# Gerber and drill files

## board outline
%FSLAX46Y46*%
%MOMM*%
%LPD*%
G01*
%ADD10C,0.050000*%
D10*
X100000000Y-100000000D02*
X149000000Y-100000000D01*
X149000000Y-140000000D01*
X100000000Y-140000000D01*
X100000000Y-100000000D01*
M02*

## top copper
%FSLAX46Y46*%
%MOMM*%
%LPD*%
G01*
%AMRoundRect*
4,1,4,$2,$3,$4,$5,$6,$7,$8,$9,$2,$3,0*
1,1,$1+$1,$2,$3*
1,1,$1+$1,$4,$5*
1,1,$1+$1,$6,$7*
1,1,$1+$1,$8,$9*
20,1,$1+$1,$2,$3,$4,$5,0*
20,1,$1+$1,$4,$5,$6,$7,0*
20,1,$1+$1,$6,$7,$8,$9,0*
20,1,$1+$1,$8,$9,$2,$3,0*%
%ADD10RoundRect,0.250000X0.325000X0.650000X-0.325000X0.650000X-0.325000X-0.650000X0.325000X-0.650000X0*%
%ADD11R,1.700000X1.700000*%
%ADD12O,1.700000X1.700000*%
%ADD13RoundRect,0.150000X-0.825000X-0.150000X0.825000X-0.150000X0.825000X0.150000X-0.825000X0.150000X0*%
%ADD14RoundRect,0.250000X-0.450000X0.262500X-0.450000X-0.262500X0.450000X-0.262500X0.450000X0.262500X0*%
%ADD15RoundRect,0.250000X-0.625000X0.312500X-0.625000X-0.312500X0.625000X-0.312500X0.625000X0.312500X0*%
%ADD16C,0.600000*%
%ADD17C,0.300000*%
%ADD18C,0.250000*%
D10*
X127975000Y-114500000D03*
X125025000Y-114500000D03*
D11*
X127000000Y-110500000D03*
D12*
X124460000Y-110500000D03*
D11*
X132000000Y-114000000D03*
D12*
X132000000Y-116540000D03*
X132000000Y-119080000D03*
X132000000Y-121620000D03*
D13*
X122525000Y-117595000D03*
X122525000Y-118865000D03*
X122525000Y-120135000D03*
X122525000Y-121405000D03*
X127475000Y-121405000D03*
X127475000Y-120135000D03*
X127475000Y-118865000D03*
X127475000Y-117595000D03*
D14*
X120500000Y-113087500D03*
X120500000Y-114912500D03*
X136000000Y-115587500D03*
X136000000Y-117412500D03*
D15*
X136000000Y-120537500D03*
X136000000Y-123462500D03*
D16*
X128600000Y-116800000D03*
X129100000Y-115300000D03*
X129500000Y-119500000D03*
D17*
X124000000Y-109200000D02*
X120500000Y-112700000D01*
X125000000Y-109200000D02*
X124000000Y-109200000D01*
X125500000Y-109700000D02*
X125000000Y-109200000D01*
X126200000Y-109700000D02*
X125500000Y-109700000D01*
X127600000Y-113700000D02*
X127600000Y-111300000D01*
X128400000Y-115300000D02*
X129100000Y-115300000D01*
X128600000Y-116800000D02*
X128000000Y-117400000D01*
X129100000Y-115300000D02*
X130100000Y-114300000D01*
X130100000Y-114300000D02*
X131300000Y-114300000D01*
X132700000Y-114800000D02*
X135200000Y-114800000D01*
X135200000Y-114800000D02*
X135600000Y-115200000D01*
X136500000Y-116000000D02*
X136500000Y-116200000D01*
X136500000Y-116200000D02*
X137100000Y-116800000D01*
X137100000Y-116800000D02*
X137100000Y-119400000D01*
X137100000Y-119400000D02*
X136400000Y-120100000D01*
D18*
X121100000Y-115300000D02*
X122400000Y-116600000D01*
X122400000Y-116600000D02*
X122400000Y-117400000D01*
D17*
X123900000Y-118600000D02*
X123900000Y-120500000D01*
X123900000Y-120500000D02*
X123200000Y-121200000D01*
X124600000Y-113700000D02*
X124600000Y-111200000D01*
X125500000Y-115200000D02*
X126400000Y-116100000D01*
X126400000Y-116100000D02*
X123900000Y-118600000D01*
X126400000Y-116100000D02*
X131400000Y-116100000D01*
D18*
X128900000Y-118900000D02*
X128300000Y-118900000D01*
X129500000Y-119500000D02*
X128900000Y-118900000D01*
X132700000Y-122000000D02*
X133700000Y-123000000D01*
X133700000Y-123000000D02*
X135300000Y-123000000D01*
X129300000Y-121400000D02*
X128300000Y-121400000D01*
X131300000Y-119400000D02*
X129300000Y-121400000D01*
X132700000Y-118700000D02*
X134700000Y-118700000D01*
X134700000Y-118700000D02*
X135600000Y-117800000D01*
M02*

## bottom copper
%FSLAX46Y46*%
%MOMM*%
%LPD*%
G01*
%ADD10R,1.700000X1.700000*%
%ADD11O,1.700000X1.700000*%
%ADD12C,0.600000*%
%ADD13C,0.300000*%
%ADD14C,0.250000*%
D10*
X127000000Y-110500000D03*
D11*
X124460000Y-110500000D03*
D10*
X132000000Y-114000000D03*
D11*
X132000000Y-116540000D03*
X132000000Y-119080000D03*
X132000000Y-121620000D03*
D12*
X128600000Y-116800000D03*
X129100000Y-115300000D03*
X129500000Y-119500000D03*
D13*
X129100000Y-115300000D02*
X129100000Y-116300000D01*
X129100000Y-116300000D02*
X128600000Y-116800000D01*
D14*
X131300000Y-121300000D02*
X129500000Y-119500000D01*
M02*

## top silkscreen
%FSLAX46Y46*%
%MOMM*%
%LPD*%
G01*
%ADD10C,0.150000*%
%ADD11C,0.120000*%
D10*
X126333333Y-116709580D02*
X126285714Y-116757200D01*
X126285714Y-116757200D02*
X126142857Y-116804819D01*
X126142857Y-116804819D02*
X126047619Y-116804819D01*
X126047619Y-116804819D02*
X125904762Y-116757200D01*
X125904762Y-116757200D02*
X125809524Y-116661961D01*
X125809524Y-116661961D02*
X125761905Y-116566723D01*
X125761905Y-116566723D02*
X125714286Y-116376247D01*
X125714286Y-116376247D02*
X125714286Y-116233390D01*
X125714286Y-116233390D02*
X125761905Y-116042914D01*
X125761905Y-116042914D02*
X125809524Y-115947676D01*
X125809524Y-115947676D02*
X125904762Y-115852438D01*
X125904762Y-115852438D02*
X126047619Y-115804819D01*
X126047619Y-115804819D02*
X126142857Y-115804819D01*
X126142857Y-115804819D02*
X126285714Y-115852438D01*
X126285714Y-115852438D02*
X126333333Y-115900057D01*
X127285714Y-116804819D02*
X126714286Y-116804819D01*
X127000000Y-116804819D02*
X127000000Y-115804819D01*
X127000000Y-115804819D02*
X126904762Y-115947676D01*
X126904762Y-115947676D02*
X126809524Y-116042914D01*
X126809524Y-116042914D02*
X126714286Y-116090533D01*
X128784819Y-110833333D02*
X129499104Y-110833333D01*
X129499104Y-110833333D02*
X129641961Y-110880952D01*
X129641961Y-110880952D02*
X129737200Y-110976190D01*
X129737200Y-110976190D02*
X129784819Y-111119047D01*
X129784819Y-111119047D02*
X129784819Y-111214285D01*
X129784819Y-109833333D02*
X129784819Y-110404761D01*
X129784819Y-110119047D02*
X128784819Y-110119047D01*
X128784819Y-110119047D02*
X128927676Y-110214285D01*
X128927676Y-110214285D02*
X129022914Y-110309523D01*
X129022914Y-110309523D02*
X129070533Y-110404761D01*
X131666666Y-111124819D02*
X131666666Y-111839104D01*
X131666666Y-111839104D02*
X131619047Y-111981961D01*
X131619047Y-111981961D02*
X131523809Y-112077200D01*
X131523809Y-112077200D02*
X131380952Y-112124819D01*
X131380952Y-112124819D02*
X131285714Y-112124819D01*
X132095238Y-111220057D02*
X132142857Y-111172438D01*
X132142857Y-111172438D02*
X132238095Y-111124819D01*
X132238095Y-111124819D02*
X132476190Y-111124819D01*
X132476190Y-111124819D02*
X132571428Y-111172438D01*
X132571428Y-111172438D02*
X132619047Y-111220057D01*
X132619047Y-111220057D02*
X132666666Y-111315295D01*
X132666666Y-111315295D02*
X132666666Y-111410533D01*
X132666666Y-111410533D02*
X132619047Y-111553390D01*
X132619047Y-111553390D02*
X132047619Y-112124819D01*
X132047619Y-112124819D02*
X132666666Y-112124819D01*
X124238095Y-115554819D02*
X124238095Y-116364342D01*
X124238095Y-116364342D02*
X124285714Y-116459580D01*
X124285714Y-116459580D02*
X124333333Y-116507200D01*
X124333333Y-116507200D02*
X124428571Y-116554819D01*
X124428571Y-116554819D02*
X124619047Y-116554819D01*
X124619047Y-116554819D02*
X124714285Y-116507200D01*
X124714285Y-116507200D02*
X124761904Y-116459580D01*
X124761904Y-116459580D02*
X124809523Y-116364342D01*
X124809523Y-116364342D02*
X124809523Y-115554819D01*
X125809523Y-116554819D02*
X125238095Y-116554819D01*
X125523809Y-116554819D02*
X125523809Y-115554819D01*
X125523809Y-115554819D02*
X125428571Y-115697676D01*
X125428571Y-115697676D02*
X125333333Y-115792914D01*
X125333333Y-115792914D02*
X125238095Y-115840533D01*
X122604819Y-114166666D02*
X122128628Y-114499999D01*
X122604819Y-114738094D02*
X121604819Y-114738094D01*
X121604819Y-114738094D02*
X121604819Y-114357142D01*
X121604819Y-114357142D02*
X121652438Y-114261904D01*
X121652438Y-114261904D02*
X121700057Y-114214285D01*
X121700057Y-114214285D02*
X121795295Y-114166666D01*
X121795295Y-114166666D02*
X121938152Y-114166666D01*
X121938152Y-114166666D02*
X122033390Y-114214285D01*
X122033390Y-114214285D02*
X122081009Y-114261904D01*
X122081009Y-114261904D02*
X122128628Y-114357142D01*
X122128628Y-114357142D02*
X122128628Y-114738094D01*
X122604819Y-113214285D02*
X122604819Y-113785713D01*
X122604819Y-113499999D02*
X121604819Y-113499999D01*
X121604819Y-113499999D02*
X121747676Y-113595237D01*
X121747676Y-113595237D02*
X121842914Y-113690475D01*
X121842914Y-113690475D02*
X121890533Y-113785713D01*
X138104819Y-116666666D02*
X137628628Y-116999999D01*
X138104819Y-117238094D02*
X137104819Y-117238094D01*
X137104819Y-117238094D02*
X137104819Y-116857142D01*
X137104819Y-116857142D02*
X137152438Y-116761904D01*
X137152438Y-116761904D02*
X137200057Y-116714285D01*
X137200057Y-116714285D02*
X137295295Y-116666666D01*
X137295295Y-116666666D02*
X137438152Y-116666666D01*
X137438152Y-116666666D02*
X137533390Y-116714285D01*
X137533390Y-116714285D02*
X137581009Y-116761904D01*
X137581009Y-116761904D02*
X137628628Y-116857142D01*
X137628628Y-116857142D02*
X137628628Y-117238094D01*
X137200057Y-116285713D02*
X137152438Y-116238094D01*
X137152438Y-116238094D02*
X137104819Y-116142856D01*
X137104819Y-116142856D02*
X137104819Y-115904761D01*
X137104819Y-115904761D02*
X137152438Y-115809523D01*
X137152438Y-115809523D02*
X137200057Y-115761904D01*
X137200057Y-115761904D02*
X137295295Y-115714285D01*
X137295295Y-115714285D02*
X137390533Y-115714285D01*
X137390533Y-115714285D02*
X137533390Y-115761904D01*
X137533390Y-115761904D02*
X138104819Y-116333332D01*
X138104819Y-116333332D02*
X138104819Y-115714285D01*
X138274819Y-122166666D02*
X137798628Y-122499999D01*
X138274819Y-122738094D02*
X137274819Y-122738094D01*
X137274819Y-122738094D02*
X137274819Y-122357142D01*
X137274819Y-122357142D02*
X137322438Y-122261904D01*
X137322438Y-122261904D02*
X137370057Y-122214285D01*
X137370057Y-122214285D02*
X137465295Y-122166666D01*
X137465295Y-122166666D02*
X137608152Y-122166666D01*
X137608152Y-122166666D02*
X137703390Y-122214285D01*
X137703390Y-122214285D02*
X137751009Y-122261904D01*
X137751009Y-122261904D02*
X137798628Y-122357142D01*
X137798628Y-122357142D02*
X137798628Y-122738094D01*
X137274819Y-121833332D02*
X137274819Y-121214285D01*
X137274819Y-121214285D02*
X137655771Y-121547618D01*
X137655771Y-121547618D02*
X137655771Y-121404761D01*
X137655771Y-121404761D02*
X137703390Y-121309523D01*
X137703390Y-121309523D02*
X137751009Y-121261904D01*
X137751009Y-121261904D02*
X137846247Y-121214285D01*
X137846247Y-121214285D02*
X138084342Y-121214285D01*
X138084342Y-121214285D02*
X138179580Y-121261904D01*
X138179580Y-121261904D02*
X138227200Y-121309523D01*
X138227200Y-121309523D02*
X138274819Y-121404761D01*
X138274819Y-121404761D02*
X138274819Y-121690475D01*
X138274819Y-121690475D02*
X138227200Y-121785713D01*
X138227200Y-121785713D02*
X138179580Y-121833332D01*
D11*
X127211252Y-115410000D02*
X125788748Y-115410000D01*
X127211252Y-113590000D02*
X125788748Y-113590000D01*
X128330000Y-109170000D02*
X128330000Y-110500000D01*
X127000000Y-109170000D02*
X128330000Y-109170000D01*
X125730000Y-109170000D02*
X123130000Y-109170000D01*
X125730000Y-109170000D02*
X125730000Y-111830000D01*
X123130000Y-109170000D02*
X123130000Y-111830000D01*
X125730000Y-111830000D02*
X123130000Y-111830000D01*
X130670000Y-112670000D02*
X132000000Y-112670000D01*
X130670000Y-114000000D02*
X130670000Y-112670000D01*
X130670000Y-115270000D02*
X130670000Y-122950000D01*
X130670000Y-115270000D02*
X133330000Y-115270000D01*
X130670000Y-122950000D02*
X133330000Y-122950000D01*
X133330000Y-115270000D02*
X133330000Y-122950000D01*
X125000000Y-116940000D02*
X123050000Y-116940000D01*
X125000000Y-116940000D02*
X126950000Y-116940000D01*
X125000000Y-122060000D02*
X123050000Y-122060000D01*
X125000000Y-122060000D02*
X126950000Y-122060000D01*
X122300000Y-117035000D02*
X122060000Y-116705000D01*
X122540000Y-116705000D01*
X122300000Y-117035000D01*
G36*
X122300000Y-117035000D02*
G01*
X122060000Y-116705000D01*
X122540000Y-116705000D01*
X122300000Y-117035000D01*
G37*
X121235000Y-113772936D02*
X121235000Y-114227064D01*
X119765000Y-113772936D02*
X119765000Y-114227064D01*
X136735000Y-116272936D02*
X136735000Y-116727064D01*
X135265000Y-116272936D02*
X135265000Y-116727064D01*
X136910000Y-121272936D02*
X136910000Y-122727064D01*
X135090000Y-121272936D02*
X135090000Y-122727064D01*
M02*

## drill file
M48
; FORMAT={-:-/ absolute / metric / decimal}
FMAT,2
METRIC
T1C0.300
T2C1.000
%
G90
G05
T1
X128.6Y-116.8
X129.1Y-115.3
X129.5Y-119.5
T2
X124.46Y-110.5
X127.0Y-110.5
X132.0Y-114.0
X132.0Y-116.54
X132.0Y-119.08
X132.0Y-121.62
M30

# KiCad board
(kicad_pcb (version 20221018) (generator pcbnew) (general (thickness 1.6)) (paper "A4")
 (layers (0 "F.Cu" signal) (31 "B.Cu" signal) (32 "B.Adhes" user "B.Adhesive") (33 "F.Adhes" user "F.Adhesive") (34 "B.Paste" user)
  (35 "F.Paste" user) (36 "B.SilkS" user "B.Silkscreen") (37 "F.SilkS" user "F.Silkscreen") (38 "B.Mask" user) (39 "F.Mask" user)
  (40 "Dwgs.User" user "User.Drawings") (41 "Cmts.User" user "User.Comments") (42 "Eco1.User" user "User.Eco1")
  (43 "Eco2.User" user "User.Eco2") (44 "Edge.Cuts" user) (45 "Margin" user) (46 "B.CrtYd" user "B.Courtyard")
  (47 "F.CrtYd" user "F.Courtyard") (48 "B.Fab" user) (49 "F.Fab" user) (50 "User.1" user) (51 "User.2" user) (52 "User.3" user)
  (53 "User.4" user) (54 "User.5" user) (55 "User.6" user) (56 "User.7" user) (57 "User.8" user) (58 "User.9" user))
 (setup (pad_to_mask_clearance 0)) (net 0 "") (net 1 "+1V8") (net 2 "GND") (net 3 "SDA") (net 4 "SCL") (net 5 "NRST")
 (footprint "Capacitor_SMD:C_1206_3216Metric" (layer "F.Cu") (at 126.5 114.5 180)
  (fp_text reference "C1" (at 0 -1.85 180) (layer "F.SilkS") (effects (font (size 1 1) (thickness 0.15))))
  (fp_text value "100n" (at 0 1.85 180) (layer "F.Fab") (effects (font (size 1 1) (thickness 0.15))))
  (fp_line (start -0.711252 -0.91) (end 0.711252 -0.91) (stroke (width 0.12) (type solid)) (layer "F.SilkS"))
  (fp_line (start -0.711252 0.91) (end 0.711252 0.91) (stroke (width 0.12) (type solid)) (layer "F.SilkS"))
  (pad "1" smd roundrect (at -1.475 0 180) (size 1.15 1.8) (layers "F.Cu" "F.Paste" "F.Mask") (roundrect_rratio 0.217391) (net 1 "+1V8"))
  (pad "2" smd roundrect (at 1.475 0 180) (size 1.15 1.8) (layers "F.Cu" "F.Paste" "F.Mask") (roundrect_rratio 0.217391) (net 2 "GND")))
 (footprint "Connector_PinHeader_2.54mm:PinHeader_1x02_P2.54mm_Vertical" (layer "F.Cu") (at 127 110.5 -90)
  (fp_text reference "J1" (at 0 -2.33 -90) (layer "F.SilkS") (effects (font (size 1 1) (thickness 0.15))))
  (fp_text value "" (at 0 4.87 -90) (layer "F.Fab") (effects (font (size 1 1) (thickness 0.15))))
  (fp_line (start -1.33 -1.33) (end 0 -1.33) (stroke (width 0.12) (type solid)) (layer "F.SilkS"))
  (fp_line (start -1.33 0) (end -1.33 -1.33) (stroke (width 0.12) (type solid)) (layer "F.SilkS"))
  (fp_line (start -1.33 1.27) (end -1.33 3.87) (stroke (width 0.12) (type solid)) (layer "F.SilkS"))
  (fp_line (start -1.33 1.27) (end 1.33 1.27) (stroke (width 0.12) (type solid)) (layer "F.SilkS"))
  (fp_line (start -1.33 3.87) (end 1.33 3.87) (stroke (width 0.12) (type solid)) (layer "F.SilkS"))
  (fp_line (start 1.33 1.27) (end 1.33 3.87) (stroke (width 0.12) (type solid)) (layer "F.SilkS"))
  (pad "1" thru_hole rect (at 0 0 270) (size 1.7 1.7) (drill 1) (layers "*.Cu" "*.Mask") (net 1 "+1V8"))
  (pad "2" thru_hole oval (at 0 2.54 270) (size 1.7 1.7) (drill 1) (layers "*.Cu" "*.Mask") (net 2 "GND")))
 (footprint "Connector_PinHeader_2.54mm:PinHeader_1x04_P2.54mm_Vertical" (layer "F.Cu") (at 132 114)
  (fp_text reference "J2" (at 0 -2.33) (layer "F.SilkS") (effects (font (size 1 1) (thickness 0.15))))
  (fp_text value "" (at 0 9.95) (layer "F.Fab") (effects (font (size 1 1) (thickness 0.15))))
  (fp_line (start -1.33 -1.33) (end 0 -1.33) (stroke (width 0.12) (type solid)) (layer "F.SilkS"))
  (fp_line (start -1.33 0) (end -1.33 -1.33) (stroke (width 0.12) (type solid)) (layer "F.SilkS"))
  (fp_line (start -1.33 1.27) (end -1.33 8.95) (stroke (width 0.12) (type solid)) (layer "F.SilkS"))
  (fp_line (start -1.33 1.27) (end 1.33 1.27) (stroke (width 0.12) (type solid)) (layer "F.SilkS"))
  (fp_line (start -1.33 8.95) (end 1.33 8.95) (stroke (width 0.12) (type solid)) (layer "F.SilkS"))
  (fp_line (start 1.33 1.27) (end 1.33 8.95) (stroke (width 0.12) (type solid)) (layer "F.SilkS"))
  (pad "1" thru_hole rect (at 0 0) (size 1.7 1.7) (drill 1) (layers "*.Cu" "*.Mask") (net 1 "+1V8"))
  (pad "2" thru_hole oval (at 0 2.54) (size 1.7 1.7) (drill 1) (layers "*.Cu" "*.Mask") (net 2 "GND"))
  (pad "3" thru_hole oval (at 0 5.08) (size 1.7 1.7) (drill 1) (layers "*.Cu" "*.Mask") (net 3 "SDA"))
  (pad "4" thru_hole oval (at 0 7.62) (size 1.7 1.7) (drill 1) (layers "*.Cu" "*.Mask") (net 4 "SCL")))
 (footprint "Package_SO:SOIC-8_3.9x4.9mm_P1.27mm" (layer "F.Cu") (at 125 119.5)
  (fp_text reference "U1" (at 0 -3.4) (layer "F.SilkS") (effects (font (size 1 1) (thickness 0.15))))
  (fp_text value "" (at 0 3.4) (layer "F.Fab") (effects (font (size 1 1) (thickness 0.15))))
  (fp_line (start 0 -2.56) (end -1.95 -2.56) (stroke (width 0.12) (type solid)) (layer "F.SilkS"))
  (fp_line (start 0 -2.56) (end 1.95 -2.56) (stroke (width 0.12) (type solid)) (layer "F.SilkS"))
  (fp_line (start 0 2.56) (end -1.95 2.56) (stroke (width 0.12) (type solid)) (layer "F.SilkS"))
  (fp_line (start 0 2.56) (end 1.95 2.56) (stroke (width 0.12) (type solid)) (layer "F.SilkS"))
  (fp_poly
   (pts (xy -2.7 -2.465) (xy -2.94 -2.795) (xy -2.46 -2.795) (xy -2.7 -2.465)) (stroke (width 0.12) (type solid)) (fill solid)
   (layer "F.SilkS"))
  (pad "1" smd roundrect (at -2.475 -1.905) (size 1.95 0.6) (layers "F.Cu" "F.Paste" "F.Mask") (roundrect_rratio 0.25) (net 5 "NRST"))
  (pad "2" smd roundrect (at -2.475 -0.635) (size 1.95 0.6) (layers "F.Cu" "F.Paste" "F.Mask") (roundrect_rratio 0.25))
  (pad "3" smd roundrect (at -2.475 0.635) (size 1.95 0.6) (layers "F.Cu" "F.Paste" "F.Mask") (roundrect_rratio 0.25))
  (pad "4" smd roundrect (at -2.475 1.905) (size 1.95 0.6) (layers "F.Cu" "F.Paste" "F.Mask") (roundrect_rratio 0.25) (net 2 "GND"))
  (pad "5" smd roundrect (at 2.475 1.905) (size 1.95 0.6) (layers "F.Cu" "F.Paste" "F.Mask") (roundrect_rratio 0.25) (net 3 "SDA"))
  (pad "6" smd roundrect (at 2.475 0.635) (size 1.95 0.6) (layers "F.Cu" "F.Paste" "F.Mask") (roundrect_rratio 0.25))
  (pad "7" smd roundrect (at 2.475 -0.635) (size 1.95 0.6) (layers "F.Cu" "F.Paste" "F.Mask") (roundrect_rratio 0.25) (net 4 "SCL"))
  (pad "8" smd roundrect (at 2.475 -1.905) (size 1.95 0.6) (layers "F.Cu" "F.Paste" "F.Mask") (roundrect_rratio 0.25) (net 1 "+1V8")))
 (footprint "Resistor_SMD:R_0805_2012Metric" (layer "F.Cu") (at 120.5 114 -90)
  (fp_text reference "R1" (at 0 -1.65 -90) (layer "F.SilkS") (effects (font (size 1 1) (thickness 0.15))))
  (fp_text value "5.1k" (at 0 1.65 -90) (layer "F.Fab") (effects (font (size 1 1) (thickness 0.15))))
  (fp_line (start -0.227064 -0.735) (end 0.227064 -0.735) (stroke (width 0.12) (type solid)) (layer "F.SilkS"))
  (fp_line (start -0.227064 0.735) (end 0.227064 0.735) (stroke (width 0.12) (type solid)) (layer "F.SilkS"))
  (pad "1" smd roundrect (at -0.9125 0 270) (size 1.025 1.4) (layers "F.Cu" "F.Paste" "F.Mask") (roundrect_rratio 0.243902) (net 1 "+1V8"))
  (pad "2" smd roundrect (at 0.9125 0 270) (size 1.025 1.4) (layers "F.Cu" "F.Paste" "F.Mask") (roundrect_rratio 0.243902) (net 5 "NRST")))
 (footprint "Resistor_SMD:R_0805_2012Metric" (layer "F.Cu") (at 136 116.5 -90)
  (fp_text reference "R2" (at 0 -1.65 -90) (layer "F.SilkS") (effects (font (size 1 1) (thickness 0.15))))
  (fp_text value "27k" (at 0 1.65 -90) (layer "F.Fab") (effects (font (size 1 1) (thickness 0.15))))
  (fp_line (start -0.227064 -0.735) (end 0.227064 -0.735) (stroke (width 0.12) (type solid)) (layer "F.SilkS"))
  (fp_line (start -0.227064 0.735) (end 0.227064 0.735) (stroke (width 0.12) (type solid)) (layer "F.SilkS"))
  (pad "1" smd roundrect (at -0.9125 0 270) (size 1.025 1.4) (layers "F.Cu" "F.Paste" "F.Mask") (roundrect_rratio 0.243902) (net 1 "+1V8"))
  (pad "2" smd roundrect (at 0.9125 0 270) (size 1.025 1.4) (layers "F.Cu" "F.Paste" "F.Mask") (roundrect_rratio 0.243902) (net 3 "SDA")))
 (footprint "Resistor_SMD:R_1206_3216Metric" (layer "F.Cu") (at 136 122 -90)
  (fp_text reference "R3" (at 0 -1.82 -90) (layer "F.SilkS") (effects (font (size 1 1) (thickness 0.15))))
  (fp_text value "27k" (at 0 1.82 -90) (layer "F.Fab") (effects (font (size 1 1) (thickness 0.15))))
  (fp_line (start -0.727064 -0.91) (end 0.727064 -0.91) (stroke (width 0.12) (type solid)) (layer "F.SilkS"))
  (fp_line (start -0.727064 0.91) (end 0.727064 0.91) (stroke (width 0.12) (type solid)) (layer "F.SilkS"))
  (pad "1" smd roundrect (at -1.4625 0 270) (size 1.125 1.75) (layers "F.Cu" "F.Paste" "F.Mask") (roundrect_rratio 0.222222) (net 1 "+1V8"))
  (pad "2" smd roundrect (at 1.4625 0 270) (size 1.125 1.75) (layers "F.Cu" "F.Paste" "F.Mask") (roundrect_rratio 0.222222) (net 4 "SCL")))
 (gr_rect (start 100 100) (end 149 140) (stroke (width 0.05) (type default)) (fill none) (layer "Edge.Cuts"))
 (segment (start 124 109.2) (end 120.5 112.7) (width 0.3) (layer "F.Cu") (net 1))
 (segment (start 125 109.2) (end 124 109.2) (width 0.3) (layer "F.Cu") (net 1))
 (segment (start 125.5 109.7) (end 125 109.2) (width 0.3) (layer "F.Cu") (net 1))
 (segment (start 126.2 109.7) (end 125.5 109.7) (width 0.3) (layer "F.Cu") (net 1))
 (segment (start 127.6 113.7) (end 127.6 111.3) (width 0.3) (layer "F.Cu") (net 1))
 (segment (start 128.4 115.3) (end 129.1 115.3) (width 0.3) (layer "F.Cu") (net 1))
 (segment (start 128.6 116.8) (end 128 117.4) (width 0.3) (layer "F.Cu") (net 1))
 (segment (start 129.1 115.3) (end 130.1 114.3) (width 0.3) (layer "F.Cu") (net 1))
 (segment (start 130.1 114.3) (end 131.3 114.3) (width 0.3) (layer "F.Cu") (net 1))
 (segment (start 132.7 114.8) (end 135.2 114.8) (width 0.3) (layer "F.Cu") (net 1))
 (segment (start 135.2 114.8) (end 135.6 115.2) (width 0.3) (layer "F.Cu") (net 1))
 (segment (start 136.5 116) (end 136.5 116.2) (width 0.3) (layer "F.Cu") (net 1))
 (segment (start 136.5 116.2) (end 137.1 116.8) (width 0.3) (layer "F.Cu") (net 1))
 (segment (start 137.1 116.8) (end 137.1 119.4) (width 0.3) (layer "F.Cu") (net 1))
 (segment (start 137.1 119.4) (end 136.4 120.1) (width 0.3) (layer "F.Cu") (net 1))
 (via (at 128.6 116.8) (size 0.6) (drill 0.3) (layers "F.Cu" "B.Cu") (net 1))
 (via (at 129.1 115.3) (size 0.6) (drill 0.3) (layers "F.Cu" "B.Cu") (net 1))
 (segment (start 121.1 115.3) (end 122.4 116.6) (width 0.25) (layer "F.Cu") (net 5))
 (segment (start 122.4 116.6) (end 122.4 117.4) (width 0.25) (layer "F.Cu") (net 5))
 (segment (start 123.9 118.6) (end 123.9 120.5) (width 0.3) (layer "F.Cu") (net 2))
 (segment (start 123.9 120.5) (end 123.2 121.2) (width 0.3) (layer "F.Cu") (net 2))
 (segment (start 124.6 113.7) (end 124.6 111.2) (width 0.3) (layer "F.Cu") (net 2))
 (segment (start 125.5 115.2) (end 126.4 116.1) (width 0.3) (layer "F.Cu") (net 2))
 (segment (start 126.4 116.1) (end 123.9 118.6) (width 0.3) (layer "F.Cu") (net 2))
 (segment (start 126.4 116.1) (end 131.4 116.1) (width 0.3) (layer "F.Cu") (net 2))
 (segment (start 128.9 118.9) (end 128.3 118.9) (width 0.25) (layer "F.Cu") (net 4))
 (segment (start 129.1 115.3) (end 129.1 116.3) (width 0.3) (layer "B.Cu") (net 1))
 (segment (start 129.1 116.3) (end 128.6 116.8) (width 0.3) (layer "B.Cu") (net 1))
 (segment (start 129.5 119.5) (end 128.9 118.9) (width 0.25) (layer "F.Cu") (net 4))
 (segment (start 132.7 122) (end 133.7 123) (width 0.25) (layer "F.Cu") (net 4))
 (segment (start 133.7 123) (end 135.3 123) (width 0.25) (layer "F.Cu") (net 4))
 (via (at 129.5 119.5) (size 0.6) (drill 0.3) (layers "F.Cu" "B.Cu") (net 4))
 (segment (start 129.3 121.4) (end 128.3 121.4) (width 0.25) (layer "F.Cu") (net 3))
 (segment (start 131.3 119.4) (end 129.3 121.4) (width 0.25) (layer "F.Cu") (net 3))
 (segment (start 131.3 121.3) (end 129.5 119.5) (width 0.25) (layer "B.Cu") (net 4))
 (segment (start 132.7 118.7) (end 134.7 118.7) (width 0.25) (layer "F.Cu") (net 3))
 (segment (start 134.7 118.7) (end 135.6 117.8) (width 0.25) (layer "F.Cu") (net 3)))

